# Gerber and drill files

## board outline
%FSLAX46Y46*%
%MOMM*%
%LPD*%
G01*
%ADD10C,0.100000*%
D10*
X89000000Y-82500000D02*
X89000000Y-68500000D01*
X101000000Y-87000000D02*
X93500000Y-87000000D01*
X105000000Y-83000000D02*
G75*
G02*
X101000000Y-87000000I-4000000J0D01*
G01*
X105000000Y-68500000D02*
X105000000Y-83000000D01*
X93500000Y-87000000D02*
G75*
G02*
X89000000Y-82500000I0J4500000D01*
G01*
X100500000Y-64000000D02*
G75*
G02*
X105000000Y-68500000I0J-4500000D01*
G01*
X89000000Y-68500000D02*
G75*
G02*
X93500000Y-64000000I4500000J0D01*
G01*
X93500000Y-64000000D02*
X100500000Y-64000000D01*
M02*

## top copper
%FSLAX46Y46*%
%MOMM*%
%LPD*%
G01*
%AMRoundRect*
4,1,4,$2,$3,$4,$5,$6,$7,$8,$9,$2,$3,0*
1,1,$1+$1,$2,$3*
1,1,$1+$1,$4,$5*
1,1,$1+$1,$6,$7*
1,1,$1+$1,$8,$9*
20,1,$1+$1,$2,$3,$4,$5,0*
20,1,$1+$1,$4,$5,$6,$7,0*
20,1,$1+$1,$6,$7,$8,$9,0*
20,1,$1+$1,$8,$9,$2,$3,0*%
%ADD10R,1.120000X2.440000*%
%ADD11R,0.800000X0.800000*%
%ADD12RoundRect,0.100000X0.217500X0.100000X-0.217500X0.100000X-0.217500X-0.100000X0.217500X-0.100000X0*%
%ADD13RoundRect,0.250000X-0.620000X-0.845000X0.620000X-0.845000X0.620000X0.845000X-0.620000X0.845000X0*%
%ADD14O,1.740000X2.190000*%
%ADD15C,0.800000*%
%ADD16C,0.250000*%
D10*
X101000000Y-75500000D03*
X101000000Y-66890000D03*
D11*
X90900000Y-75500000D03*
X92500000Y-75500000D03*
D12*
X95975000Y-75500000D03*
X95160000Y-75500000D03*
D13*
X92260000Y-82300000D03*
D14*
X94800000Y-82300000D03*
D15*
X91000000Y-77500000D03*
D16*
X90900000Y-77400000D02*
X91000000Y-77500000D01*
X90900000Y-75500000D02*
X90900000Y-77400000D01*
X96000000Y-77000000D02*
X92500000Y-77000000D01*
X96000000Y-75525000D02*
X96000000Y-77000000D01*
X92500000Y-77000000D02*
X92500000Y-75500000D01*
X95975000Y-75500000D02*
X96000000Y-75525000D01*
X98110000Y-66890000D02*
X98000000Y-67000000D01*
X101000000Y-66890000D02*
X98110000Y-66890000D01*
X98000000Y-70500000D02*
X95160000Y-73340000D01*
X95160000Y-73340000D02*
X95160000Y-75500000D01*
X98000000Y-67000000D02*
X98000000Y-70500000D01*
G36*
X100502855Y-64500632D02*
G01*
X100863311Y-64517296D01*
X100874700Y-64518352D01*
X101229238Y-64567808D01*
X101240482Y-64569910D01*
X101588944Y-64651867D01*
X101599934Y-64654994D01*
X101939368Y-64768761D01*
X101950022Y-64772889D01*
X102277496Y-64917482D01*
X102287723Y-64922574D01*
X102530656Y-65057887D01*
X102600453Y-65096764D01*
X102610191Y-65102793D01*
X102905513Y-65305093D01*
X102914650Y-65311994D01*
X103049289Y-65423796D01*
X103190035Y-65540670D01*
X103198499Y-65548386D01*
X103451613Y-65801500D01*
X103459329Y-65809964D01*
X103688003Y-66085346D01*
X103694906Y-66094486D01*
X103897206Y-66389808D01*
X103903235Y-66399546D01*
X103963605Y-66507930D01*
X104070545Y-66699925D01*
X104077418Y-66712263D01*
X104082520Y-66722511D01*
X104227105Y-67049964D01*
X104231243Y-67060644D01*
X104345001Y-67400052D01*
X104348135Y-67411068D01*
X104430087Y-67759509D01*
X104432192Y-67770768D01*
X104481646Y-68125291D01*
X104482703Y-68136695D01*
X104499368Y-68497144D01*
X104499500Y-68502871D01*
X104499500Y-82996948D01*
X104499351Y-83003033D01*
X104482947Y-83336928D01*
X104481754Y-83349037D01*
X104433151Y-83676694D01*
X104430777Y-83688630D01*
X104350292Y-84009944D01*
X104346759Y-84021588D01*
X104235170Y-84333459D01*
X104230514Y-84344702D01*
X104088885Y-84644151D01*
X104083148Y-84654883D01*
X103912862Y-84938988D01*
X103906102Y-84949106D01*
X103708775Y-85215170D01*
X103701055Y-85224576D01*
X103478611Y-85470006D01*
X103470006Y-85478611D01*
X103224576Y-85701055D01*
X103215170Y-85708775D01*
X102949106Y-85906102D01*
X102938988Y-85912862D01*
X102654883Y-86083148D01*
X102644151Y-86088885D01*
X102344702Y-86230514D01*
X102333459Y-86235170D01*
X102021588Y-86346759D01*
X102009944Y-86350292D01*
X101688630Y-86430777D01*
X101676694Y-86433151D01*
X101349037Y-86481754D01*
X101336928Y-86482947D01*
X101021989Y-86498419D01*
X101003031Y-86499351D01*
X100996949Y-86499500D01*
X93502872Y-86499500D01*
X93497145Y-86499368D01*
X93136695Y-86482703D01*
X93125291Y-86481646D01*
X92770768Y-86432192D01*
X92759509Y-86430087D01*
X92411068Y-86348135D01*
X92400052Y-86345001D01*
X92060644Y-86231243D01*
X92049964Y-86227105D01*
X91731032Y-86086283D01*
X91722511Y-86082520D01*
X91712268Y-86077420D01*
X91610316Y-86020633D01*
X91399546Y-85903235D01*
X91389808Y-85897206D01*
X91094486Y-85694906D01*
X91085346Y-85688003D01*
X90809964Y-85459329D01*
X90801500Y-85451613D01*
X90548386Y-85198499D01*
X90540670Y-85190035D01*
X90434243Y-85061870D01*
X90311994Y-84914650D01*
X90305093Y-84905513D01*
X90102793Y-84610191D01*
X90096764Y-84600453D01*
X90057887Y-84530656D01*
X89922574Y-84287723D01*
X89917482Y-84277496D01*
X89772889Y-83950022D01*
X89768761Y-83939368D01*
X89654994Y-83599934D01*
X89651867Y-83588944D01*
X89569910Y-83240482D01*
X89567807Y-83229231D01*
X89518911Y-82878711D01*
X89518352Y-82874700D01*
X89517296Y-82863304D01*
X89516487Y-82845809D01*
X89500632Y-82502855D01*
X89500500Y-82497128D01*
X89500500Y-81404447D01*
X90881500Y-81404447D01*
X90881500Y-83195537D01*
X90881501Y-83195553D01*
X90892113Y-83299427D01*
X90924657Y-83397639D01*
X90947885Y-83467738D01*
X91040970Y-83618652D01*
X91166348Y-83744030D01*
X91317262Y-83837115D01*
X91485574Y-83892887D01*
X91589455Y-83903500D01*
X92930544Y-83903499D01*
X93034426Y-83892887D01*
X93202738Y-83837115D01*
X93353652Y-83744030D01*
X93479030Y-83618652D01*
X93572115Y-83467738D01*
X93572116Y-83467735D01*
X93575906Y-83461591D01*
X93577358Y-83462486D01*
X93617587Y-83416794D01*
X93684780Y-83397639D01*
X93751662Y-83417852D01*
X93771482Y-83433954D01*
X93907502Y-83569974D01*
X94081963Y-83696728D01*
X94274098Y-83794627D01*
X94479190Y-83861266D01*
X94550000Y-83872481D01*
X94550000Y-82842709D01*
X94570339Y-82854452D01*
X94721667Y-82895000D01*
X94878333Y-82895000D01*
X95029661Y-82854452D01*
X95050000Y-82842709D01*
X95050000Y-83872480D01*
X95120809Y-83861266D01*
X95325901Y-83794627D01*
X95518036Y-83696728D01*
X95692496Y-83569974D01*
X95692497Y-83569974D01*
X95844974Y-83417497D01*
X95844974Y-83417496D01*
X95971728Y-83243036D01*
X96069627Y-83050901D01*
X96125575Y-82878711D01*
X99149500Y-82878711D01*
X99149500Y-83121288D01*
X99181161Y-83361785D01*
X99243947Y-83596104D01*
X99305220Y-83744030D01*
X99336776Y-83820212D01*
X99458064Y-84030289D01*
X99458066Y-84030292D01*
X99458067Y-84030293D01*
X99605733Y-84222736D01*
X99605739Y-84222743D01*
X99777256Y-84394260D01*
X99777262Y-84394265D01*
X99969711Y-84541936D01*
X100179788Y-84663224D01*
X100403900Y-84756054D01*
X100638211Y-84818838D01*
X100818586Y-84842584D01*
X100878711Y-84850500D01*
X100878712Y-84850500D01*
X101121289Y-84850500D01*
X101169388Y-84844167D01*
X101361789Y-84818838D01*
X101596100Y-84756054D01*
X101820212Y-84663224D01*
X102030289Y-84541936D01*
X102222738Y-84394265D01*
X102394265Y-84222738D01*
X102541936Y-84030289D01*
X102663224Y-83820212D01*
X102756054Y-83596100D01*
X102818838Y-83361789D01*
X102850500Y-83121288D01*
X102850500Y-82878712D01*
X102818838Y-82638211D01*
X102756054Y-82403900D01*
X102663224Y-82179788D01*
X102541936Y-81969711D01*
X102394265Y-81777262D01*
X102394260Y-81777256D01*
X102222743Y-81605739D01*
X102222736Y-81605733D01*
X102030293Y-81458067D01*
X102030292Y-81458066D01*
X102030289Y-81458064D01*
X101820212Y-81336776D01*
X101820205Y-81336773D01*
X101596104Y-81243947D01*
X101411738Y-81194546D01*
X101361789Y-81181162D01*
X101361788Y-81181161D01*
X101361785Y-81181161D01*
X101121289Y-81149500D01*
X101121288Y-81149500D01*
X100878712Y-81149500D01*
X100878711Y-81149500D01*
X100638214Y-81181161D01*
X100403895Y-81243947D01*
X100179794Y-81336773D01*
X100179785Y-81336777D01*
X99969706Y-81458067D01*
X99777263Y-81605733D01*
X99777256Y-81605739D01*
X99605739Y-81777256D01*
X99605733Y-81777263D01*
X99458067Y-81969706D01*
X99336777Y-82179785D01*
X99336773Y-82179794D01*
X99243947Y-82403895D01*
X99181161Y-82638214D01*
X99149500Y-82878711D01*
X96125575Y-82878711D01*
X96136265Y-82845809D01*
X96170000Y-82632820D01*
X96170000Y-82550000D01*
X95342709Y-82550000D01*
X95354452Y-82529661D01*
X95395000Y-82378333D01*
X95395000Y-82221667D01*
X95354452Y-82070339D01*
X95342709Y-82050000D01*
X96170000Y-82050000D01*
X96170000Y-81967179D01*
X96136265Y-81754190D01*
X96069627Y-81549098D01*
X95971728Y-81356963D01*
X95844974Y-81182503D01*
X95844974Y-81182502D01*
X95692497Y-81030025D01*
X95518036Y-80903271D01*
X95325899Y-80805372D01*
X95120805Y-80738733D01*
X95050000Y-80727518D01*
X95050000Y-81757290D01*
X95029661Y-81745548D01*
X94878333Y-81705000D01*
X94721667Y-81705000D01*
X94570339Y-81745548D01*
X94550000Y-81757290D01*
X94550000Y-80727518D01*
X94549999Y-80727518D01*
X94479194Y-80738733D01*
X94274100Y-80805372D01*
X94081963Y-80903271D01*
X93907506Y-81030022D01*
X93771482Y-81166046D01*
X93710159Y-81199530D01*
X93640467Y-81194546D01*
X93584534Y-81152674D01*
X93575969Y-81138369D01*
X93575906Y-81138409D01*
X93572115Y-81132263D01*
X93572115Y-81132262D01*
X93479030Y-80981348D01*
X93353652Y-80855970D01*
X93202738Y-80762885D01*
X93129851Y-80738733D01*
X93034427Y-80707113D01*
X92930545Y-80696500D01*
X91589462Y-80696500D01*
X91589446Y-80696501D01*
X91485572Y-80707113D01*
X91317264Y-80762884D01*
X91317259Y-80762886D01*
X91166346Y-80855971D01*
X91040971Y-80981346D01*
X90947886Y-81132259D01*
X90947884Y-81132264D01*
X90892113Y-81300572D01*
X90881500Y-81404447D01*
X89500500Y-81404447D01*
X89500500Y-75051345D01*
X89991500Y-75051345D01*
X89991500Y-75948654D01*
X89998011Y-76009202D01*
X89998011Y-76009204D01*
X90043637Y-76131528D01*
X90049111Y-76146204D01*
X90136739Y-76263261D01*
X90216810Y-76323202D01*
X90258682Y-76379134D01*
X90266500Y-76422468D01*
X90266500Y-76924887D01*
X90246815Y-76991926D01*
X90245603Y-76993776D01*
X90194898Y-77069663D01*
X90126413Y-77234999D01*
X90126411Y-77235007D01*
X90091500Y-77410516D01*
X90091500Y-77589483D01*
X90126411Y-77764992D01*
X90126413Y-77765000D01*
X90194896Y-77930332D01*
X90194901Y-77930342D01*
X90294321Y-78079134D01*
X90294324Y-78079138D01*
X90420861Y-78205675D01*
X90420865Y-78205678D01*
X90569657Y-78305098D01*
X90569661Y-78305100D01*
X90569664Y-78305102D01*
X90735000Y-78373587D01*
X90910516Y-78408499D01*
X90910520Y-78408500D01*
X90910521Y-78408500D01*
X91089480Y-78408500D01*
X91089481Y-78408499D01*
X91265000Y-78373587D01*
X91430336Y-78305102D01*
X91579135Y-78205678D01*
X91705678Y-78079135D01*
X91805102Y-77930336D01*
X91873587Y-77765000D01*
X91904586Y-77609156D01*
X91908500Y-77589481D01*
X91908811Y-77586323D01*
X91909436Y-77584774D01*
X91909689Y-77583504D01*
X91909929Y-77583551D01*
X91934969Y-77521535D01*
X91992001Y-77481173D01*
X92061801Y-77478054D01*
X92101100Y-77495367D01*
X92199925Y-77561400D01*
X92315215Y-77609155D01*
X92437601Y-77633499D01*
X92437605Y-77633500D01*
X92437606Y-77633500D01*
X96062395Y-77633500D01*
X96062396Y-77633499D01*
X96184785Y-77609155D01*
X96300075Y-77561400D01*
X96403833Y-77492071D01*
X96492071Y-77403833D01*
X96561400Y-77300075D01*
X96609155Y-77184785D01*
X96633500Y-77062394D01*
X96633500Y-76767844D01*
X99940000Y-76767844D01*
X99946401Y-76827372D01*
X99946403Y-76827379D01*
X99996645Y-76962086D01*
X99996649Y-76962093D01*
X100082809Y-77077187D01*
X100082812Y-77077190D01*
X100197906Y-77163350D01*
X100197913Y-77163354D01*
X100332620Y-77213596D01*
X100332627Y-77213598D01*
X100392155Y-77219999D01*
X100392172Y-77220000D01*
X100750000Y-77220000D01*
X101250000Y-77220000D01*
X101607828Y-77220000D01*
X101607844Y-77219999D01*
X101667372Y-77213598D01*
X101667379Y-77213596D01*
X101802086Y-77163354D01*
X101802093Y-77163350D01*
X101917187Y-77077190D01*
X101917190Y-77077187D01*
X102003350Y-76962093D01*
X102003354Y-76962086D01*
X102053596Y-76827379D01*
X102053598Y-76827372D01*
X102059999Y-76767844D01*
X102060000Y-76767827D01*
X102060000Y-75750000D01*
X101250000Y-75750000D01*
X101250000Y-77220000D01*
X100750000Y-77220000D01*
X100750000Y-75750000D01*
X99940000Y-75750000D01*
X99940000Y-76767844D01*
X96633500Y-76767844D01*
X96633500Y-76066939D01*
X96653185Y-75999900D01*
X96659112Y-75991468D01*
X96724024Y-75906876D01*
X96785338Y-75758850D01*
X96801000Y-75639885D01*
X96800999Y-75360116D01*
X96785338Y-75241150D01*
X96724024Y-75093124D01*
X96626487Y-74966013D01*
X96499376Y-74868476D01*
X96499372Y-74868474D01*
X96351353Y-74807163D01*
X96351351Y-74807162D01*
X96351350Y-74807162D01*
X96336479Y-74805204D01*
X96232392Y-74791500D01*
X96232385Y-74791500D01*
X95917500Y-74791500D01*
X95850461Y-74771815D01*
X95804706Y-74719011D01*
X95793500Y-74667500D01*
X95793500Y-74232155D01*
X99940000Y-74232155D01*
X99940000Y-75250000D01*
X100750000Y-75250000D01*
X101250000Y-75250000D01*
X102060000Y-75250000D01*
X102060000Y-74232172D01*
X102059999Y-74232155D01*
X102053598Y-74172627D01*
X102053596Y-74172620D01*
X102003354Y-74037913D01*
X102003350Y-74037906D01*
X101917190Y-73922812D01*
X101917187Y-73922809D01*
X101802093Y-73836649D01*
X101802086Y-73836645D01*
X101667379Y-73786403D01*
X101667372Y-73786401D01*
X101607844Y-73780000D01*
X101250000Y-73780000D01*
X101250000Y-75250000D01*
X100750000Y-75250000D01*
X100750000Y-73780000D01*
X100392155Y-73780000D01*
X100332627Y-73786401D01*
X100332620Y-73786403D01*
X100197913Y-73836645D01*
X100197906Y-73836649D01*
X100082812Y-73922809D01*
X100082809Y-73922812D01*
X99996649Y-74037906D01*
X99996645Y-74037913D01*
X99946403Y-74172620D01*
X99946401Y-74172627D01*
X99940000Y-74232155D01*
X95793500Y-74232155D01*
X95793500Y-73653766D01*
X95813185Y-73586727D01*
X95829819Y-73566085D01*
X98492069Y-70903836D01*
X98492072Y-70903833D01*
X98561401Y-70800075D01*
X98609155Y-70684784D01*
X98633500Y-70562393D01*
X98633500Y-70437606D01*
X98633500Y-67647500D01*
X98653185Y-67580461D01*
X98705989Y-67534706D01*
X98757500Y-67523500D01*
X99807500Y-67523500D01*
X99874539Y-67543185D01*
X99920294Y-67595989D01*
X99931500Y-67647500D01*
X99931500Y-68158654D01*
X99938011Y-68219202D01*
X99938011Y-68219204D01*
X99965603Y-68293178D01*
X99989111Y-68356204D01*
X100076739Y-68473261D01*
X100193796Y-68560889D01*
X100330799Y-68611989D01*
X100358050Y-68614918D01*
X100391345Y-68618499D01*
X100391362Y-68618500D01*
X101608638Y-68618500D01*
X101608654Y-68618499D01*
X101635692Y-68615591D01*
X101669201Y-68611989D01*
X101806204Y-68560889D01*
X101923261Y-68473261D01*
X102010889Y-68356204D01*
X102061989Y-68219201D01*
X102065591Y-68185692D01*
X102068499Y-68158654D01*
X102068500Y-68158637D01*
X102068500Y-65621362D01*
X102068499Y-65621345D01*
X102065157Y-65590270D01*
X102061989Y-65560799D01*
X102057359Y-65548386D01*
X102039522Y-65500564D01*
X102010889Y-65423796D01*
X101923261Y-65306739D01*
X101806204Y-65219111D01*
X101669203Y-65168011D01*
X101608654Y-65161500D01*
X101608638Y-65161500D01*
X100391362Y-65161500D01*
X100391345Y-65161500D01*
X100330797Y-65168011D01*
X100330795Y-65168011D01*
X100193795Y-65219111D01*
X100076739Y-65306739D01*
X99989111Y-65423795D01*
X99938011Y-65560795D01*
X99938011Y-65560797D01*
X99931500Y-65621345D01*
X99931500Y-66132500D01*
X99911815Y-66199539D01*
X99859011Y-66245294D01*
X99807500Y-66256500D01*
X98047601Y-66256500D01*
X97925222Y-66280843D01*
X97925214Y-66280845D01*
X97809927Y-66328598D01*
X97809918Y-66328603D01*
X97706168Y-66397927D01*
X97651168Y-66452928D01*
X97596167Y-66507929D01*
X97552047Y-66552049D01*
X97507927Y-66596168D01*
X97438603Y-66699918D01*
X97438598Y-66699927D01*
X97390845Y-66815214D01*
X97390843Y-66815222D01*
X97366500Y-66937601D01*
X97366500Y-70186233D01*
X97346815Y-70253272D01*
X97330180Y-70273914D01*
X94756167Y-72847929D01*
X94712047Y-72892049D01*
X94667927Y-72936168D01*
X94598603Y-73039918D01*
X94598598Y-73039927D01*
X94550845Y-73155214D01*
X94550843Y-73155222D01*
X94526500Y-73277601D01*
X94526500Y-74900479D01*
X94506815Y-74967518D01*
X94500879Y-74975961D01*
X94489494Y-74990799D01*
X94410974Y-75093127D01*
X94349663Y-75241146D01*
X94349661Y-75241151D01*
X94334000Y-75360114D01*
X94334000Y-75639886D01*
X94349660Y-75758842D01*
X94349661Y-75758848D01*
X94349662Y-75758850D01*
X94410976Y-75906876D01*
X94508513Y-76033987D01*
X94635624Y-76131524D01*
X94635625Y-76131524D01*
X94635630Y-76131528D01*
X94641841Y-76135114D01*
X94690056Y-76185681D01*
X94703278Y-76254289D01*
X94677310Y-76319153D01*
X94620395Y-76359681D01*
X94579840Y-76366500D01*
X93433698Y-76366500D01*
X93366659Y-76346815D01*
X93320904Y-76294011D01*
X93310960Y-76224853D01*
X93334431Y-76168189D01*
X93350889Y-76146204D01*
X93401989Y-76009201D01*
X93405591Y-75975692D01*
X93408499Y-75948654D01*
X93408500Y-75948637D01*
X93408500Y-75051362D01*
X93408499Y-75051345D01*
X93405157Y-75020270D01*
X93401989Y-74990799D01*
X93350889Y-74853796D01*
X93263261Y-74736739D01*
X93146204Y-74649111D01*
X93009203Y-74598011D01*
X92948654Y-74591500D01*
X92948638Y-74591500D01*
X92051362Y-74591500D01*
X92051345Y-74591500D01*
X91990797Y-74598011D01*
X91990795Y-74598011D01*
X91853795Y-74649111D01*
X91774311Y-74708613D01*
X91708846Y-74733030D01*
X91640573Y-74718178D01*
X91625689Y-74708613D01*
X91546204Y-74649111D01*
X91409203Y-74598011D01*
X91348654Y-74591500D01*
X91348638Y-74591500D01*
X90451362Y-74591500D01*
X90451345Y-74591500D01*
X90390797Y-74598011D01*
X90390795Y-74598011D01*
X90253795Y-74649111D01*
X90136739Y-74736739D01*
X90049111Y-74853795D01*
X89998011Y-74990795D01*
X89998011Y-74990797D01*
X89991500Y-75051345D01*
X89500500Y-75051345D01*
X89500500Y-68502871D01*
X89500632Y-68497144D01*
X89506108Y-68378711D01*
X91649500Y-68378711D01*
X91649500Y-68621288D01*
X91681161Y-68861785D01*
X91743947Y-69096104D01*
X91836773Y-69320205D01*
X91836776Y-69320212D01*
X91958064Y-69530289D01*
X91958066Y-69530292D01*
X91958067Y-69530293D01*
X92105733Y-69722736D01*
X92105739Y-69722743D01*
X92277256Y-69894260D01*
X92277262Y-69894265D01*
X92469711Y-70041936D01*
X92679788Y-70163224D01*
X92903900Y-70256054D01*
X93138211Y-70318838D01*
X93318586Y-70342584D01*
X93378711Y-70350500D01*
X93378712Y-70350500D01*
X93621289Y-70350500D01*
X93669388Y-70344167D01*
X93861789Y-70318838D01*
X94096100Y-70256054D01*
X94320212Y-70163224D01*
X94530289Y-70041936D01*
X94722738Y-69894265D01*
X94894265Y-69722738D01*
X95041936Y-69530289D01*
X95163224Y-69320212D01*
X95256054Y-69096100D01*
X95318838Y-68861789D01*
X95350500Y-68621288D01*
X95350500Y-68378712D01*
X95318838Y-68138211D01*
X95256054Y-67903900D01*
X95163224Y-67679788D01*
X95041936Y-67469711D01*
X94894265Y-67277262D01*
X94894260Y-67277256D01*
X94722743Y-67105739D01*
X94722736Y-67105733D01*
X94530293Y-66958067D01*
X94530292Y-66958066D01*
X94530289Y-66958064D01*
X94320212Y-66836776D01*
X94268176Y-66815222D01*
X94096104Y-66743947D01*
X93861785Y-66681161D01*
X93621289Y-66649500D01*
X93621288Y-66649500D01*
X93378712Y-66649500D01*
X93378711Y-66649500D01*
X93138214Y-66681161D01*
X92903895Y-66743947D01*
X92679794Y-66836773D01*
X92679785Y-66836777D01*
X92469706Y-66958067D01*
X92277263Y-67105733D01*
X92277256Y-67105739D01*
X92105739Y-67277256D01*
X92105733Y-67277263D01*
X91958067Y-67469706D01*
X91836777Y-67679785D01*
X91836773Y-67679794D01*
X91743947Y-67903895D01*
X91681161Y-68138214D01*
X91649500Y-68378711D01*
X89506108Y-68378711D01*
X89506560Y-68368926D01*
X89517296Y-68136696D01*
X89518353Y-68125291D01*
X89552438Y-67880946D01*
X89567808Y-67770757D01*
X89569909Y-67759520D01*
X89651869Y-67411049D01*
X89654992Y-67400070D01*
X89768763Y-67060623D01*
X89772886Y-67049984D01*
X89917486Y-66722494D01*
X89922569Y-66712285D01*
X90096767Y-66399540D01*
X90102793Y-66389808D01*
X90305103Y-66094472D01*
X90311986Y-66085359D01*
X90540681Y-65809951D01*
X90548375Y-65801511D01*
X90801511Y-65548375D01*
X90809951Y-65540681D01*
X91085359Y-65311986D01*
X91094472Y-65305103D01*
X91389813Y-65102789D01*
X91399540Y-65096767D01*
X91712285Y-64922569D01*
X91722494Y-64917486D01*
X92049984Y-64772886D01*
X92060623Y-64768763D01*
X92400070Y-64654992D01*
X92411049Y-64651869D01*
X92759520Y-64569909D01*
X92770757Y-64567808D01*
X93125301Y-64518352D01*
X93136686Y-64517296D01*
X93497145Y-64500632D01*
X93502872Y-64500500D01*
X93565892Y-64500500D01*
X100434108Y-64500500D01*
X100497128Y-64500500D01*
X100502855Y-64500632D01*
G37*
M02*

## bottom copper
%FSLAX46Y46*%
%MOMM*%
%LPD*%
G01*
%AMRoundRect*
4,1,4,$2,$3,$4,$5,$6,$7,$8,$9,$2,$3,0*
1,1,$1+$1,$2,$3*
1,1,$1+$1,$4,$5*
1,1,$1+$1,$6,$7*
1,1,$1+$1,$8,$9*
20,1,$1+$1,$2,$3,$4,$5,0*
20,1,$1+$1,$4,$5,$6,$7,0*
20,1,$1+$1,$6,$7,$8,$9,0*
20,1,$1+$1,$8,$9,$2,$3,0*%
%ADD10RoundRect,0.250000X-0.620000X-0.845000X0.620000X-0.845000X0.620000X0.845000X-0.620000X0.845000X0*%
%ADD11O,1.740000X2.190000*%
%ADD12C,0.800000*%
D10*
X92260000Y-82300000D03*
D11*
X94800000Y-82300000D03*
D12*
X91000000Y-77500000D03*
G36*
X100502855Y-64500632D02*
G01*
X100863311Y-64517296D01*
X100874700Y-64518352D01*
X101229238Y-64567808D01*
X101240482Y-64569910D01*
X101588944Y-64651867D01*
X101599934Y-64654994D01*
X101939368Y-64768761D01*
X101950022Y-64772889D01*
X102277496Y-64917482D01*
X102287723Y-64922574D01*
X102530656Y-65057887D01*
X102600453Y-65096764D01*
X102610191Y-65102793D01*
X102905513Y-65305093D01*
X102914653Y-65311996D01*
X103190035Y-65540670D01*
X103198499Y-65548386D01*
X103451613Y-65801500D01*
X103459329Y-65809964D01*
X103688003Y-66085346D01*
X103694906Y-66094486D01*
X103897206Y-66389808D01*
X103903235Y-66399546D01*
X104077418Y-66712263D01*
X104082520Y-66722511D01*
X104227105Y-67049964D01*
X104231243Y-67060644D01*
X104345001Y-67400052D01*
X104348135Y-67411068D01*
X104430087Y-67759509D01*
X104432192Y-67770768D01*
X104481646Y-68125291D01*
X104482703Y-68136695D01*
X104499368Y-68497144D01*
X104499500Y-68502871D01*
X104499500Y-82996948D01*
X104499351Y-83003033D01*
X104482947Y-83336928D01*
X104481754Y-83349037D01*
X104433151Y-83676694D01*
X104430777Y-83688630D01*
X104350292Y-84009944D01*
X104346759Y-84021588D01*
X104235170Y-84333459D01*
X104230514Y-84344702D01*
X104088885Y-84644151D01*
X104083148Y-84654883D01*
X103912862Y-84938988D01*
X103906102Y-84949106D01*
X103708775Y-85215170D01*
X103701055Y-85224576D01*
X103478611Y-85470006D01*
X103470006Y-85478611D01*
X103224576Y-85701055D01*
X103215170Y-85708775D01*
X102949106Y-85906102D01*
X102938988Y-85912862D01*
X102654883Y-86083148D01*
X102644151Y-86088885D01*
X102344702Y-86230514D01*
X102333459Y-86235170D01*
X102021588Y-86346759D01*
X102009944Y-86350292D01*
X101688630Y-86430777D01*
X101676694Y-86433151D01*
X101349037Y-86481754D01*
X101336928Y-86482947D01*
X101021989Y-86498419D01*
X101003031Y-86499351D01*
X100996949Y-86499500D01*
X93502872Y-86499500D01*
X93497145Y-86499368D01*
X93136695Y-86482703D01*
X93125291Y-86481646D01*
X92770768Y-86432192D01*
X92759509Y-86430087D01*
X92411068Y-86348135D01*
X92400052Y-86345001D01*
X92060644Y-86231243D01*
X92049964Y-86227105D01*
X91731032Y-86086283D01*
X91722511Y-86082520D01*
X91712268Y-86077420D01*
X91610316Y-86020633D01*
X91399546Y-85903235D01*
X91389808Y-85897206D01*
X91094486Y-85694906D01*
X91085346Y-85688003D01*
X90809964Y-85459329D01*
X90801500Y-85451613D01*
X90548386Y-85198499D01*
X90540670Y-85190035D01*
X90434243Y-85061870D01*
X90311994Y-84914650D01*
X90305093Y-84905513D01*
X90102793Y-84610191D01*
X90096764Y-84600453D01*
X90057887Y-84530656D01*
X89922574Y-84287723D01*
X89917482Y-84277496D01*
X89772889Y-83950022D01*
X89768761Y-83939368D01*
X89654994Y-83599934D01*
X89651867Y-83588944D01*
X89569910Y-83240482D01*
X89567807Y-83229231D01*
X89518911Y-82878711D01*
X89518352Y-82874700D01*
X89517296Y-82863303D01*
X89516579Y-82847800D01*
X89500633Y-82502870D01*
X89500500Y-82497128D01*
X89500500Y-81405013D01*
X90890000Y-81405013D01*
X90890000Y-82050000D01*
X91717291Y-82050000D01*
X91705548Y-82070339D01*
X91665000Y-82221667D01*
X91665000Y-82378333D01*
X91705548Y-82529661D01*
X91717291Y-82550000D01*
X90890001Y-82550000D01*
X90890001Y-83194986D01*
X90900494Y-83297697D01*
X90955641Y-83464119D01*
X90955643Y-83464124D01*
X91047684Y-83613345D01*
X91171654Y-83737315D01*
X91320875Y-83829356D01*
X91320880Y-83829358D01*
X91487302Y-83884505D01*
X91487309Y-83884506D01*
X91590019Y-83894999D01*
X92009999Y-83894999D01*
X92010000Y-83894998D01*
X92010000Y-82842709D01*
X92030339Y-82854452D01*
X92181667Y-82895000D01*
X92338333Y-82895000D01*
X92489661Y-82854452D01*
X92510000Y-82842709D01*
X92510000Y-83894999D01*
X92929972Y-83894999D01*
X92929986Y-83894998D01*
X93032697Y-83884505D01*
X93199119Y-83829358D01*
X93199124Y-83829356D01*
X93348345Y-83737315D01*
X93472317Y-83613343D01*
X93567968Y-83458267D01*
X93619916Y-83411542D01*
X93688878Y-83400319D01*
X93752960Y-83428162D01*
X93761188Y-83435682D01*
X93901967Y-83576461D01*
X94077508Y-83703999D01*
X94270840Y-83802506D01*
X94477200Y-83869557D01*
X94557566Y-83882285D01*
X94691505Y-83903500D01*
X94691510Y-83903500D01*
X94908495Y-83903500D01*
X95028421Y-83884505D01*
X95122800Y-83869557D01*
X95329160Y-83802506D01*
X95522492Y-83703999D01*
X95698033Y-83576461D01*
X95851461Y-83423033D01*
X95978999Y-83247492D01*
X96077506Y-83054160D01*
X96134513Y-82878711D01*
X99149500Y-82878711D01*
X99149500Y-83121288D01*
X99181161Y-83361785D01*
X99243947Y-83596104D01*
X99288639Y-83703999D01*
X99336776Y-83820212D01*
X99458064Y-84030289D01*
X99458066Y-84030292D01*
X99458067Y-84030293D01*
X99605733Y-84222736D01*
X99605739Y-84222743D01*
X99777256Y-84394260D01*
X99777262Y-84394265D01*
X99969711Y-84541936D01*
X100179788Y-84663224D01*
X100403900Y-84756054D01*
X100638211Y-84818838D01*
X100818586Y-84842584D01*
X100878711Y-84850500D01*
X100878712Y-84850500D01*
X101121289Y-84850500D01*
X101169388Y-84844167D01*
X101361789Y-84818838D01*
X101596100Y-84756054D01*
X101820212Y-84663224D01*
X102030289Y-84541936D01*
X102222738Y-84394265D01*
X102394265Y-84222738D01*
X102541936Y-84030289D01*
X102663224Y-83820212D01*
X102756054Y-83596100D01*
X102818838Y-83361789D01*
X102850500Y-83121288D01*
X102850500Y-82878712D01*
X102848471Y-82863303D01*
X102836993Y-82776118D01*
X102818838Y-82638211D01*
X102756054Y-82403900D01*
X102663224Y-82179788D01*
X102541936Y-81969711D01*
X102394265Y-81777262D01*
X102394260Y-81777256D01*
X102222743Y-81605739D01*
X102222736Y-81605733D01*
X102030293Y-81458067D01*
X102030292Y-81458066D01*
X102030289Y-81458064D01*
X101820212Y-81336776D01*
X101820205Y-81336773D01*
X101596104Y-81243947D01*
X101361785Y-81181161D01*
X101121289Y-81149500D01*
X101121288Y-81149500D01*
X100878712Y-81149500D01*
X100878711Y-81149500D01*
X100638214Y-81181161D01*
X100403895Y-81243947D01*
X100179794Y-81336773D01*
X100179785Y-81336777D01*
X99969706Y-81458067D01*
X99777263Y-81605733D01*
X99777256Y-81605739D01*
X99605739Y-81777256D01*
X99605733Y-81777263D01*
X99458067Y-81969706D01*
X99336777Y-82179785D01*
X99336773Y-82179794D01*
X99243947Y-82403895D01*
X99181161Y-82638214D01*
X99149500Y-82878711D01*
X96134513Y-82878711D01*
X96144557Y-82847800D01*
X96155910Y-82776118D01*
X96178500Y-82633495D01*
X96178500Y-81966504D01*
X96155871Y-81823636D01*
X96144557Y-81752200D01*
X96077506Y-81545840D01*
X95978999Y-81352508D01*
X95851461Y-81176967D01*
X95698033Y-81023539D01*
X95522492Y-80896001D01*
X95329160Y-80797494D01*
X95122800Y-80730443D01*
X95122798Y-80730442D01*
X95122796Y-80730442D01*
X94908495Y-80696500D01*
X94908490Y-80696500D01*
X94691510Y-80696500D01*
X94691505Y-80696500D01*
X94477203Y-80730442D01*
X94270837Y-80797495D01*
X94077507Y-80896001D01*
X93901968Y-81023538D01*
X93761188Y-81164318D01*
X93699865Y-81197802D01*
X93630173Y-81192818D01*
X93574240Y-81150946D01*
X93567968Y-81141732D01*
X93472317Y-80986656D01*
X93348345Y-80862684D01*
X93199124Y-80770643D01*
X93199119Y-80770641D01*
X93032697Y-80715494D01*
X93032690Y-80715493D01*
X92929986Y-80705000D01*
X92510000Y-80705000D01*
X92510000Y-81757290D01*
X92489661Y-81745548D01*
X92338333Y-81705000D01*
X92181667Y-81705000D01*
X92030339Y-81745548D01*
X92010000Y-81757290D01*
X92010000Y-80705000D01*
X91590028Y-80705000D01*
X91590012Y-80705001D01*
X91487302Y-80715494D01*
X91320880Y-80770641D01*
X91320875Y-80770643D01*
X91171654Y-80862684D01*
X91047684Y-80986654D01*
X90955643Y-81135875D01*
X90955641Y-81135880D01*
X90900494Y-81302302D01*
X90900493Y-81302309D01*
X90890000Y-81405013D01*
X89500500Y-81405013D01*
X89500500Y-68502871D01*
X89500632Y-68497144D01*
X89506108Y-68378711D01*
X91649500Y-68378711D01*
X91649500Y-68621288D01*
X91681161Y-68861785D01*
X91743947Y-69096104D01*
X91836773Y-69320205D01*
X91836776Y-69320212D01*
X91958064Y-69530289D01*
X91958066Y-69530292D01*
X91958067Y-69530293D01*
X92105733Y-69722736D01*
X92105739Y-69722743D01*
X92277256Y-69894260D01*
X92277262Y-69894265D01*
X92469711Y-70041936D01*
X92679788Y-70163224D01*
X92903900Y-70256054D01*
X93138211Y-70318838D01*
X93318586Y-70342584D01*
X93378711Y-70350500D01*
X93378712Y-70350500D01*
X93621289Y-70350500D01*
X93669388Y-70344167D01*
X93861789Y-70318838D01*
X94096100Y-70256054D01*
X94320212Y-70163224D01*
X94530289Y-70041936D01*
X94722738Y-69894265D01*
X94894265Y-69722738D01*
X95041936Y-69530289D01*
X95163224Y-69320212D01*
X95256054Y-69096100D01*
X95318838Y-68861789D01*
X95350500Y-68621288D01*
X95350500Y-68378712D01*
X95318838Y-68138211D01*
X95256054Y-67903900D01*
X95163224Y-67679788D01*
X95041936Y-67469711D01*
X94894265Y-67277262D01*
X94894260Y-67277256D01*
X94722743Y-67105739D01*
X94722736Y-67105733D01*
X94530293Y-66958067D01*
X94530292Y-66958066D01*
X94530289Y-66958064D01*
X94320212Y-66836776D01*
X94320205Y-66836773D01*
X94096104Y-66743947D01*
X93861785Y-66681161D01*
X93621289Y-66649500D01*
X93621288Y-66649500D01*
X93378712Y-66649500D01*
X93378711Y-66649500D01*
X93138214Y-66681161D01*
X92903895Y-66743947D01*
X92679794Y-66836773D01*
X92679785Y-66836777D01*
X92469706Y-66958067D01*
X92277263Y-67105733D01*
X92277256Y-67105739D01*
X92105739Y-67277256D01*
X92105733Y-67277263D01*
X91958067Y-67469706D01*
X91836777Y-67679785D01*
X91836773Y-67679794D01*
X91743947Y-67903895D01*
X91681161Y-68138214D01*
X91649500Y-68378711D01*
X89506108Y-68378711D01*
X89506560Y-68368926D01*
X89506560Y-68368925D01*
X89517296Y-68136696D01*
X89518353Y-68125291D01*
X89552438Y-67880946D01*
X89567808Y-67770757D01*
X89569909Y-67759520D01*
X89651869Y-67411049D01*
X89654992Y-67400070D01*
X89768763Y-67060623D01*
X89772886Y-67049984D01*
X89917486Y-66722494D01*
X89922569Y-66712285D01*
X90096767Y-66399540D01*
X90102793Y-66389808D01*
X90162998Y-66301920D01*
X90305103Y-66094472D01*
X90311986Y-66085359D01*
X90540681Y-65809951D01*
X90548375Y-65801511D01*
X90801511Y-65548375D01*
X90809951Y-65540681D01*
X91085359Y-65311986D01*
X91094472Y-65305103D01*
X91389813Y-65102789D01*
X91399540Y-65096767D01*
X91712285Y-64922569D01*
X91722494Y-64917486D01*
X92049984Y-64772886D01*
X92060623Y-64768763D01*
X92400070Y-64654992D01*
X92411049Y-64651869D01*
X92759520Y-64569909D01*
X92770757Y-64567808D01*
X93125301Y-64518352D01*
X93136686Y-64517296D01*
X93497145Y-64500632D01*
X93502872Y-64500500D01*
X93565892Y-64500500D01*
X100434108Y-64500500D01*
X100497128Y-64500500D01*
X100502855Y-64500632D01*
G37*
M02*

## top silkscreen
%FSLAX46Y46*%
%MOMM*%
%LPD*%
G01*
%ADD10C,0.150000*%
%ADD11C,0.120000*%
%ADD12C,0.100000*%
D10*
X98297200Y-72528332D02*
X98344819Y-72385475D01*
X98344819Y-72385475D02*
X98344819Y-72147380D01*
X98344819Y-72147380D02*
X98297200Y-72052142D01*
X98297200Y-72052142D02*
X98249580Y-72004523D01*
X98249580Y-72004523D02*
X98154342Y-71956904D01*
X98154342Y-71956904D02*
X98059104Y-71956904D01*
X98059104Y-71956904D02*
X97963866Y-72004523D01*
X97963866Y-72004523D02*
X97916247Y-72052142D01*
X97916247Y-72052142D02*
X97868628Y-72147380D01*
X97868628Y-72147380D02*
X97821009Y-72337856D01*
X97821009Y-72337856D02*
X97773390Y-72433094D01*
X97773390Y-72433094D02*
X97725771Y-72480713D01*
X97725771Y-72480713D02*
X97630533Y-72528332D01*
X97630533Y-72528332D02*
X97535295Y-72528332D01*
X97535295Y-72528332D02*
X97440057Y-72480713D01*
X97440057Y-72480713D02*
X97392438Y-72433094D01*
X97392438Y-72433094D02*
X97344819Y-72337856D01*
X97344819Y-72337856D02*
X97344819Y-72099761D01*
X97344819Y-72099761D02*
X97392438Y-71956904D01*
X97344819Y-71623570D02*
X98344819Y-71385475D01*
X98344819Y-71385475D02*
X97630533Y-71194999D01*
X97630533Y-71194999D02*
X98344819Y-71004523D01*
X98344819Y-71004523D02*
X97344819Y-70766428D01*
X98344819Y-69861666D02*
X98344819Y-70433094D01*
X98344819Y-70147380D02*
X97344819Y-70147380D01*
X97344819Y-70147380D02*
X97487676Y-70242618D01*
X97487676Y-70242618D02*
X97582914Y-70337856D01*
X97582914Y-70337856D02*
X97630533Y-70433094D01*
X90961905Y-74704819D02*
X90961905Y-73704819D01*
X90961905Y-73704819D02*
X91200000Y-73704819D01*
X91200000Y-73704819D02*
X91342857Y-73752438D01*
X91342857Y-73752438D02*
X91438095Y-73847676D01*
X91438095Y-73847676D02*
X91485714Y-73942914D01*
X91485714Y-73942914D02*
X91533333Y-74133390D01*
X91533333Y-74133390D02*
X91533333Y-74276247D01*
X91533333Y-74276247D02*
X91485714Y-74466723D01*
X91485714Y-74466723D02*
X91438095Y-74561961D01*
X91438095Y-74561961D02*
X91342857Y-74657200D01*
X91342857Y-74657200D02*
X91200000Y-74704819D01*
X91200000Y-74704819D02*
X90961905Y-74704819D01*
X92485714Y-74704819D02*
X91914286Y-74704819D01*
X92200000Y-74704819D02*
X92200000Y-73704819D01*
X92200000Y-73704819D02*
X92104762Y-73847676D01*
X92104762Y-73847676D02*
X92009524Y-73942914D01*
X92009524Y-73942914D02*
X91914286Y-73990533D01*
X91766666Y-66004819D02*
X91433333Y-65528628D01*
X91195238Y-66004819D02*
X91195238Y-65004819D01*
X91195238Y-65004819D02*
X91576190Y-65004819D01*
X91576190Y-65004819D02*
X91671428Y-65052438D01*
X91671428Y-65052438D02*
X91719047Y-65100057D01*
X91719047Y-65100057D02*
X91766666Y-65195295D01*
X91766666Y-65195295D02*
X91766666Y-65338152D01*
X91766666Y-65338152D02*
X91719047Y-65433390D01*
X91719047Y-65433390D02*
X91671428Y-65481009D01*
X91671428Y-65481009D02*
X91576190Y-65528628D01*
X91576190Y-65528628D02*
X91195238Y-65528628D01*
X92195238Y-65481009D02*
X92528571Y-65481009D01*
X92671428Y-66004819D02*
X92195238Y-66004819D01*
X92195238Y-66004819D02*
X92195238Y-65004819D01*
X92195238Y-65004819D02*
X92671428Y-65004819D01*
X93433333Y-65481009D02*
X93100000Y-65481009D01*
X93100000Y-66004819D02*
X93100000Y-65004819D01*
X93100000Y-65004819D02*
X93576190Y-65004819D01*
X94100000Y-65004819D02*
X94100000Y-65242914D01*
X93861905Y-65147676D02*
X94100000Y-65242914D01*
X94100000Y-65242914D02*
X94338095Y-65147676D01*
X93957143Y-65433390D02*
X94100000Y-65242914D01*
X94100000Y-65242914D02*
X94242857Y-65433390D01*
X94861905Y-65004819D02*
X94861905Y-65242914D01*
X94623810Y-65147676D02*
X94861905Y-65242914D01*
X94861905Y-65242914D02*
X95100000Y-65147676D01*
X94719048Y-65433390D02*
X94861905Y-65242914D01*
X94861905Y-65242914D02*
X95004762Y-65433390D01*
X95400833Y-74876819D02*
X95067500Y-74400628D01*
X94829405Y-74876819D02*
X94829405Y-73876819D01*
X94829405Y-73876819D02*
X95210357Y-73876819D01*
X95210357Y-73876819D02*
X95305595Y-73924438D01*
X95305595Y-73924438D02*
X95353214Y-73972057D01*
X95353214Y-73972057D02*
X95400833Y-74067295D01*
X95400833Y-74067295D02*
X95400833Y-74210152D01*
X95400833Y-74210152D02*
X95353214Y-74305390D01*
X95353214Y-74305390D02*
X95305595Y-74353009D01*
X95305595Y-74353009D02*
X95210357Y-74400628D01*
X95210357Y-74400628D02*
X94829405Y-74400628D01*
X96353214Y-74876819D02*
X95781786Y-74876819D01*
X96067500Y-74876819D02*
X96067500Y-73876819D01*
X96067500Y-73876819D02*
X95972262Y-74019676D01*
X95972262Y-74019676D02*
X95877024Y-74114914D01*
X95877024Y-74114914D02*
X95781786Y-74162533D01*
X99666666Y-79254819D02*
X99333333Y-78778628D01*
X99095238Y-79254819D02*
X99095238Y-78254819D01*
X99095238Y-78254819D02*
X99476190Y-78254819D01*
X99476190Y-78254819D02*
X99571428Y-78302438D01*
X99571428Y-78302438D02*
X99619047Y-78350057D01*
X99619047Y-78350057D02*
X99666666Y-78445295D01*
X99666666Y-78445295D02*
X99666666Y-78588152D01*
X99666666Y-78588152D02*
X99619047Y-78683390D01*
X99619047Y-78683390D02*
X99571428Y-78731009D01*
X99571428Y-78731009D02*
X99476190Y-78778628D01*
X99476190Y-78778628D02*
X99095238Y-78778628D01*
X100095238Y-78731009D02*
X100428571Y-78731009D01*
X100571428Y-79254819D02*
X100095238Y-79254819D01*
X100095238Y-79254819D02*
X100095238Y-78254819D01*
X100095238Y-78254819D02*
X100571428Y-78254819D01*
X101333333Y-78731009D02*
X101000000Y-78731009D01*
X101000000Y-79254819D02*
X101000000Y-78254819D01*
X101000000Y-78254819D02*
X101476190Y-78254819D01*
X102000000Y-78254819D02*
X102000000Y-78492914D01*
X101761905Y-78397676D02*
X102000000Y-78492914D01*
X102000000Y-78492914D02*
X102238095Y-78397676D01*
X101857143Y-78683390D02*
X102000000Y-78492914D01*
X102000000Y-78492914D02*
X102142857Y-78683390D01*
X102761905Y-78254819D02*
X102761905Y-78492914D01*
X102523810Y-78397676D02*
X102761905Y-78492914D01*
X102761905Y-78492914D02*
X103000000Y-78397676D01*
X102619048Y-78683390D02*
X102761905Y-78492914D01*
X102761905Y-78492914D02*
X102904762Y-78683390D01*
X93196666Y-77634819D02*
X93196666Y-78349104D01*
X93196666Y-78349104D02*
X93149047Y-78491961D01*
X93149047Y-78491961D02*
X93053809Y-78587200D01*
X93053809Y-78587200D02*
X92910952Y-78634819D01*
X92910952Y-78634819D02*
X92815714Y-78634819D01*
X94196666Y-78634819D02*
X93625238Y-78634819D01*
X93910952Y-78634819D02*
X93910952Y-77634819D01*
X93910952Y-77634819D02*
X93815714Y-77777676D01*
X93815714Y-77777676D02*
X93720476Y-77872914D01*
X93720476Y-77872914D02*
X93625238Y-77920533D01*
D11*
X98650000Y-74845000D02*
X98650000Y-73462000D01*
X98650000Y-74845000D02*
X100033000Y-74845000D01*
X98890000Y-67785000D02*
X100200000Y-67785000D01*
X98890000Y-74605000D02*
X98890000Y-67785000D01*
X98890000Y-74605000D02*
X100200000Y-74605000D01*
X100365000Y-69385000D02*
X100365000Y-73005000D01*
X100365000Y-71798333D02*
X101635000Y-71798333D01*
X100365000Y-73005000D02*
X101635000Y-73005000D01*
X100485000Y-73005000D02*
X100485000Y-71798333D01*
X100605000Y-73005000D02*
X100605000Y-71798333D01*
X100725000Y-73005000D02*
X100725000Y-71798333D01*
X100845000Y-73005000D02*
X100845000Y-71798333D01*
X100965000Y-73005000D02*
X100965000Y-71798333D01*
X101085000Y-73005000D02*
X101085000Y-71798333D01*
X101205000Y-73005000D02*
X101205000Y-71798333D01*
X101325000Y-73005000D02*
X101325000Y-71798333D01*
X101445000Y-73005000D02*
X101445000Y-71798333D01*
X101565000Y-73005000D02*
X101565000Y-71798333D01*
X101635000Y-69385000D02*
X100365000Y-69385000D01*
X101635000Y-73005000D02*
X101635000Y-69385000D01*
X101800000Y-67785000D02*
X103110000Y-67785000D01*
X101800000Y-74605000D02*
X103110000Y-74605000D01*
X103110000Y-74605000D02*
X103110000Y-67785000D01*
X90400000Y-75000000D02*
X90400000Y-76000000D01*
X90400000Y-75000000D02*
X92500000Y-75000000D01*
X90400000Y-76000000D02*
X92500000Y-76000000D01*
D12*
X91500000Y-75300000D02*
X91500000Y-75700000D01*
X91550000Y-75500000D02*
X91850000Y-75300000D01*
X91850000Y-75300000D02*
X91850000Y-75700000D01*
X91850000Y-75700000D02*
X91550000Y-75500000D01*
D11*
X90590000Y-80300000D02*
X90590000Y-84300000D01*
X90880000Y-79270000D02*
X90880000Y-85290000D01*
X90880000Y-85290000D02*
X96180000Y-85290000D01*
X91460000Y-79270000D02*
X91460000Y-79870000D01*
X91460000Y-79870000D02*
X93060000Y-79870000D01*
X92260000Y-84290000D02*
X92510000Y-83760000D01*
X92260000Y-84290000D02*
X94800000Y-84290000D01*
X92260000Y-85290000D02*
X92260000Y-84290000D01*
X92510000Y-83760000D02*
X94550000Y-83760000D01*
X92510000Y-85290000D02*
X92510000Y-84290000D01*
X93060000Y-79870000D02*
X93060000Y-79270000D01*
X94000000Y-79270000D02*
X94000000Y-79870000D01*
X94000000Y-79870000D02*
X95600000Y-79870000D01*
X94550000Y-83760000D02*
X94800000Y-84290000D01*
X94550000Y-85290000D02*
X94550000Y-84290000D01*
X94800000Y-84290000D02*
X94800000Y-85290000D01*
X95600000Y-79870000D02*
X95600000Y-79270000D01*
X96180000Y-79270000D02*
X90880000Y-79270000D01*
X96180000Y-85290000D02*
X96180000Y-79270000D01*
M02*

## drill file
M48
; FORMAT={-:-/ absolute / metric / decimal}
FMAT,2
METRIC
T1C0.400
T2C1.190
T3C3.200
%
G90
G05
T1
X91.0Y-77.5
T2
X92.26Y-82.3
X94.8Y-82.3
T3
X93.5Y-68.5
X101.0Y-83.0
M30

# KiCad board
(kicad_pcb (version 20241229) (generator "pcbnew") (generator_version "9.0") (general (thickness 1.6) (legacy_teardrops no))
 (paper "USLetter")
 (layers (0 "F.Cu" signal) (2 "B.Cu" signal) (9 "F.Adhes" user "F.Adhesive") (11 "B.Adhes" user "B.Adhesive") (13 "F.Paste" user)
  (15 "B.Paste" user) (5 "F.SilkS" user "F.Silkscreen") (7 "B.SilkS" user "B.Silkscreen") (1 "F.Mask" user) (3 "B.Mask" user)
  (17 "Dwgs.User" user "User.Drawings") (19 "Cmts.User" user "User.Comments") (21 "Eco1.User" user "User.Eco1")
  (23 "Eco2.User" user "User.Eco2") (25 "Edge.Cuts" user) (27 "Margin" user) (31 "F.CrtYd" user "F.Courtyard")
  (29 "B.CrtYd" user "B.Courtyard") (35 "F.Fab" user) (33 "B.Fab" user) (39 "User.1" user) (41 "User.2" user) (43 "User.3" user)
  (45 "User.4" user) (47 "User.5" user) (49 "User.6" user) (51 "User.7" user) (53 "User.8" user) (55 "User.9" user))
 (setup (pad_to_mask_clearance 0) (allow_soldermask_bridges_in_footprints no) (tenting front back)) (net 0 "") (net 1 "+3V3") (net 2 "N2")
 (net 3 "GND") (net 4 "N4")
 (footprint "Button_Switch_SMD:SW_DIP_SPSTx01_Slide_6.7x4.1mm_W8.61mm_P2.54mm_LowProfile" (layer "F.Cu") (at 101 71.195 90)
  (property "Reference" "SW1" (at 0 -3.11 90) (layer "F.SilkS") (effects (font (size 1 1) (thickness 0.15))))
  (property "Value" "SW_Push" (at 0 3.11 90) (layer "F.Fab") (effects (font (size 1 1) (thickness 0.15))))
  (fp_line (start -3.65 -2.35) (end -2.267 -2.35) (stroke (width 0.12) (type solid)) (layer "F.SilkS"))
  (fp_line (start -3.65 -2.35) (end -3.65 -0.967) (stroke (width 0.12) (type solid)) (layer "F.SilkS"))
  (fp_line (start 3.41 -2.11) (end 3.41 -0.8) (stroke (width 0.12) (type solid)) (layer "F.SilkS"))
  (fp_line (start -3.41 -2.11) (end 3.41 -2.11) (stroke (width 0.12) (type solid)) (layer "F.SilkS"))
  (fp_line (start -3.41 -2.11) (end -3.41 -0.8) (stroke (width 0.12) (type solid)) (layer "F.SilkS"))
  (fp_line (start 1.81 -0.635) (end -1.81 -0.635) (stroke (width 0.12) (type solid)) (layer "F.SilkS"))
  (fp_line (start -0.603333 -0.635) (end -0.603333 0.635) (stroke (width 0.12) (type solid)) (layer "F.SilkS"))
  (fp_line (start -1.81 -0.635) (end -1.81 0.635) (stroke (width 0.12) (type solid)) (layer "F.SilkS"))
  (fp_line (start -1.81 -0.515) (end -0.603333 -0.515) (stroke (width 0.12) (type solid)) (layer "F.SilkS"))
  (fp_line (start -1.81 -0.395) (end -0.603333 -0.395) (stroke (width 0.12) (type solid)) (layer "F.SilkS"))
  (fp_line (start -1.81 -0.275) (end -0.603333 -0.275) (stroke (width 0.12) (type solid)) (layer "F.SilkS"))
  (fp_line (start -1.81 -0.155) (end -0.603333 -0.155) (stroke (width 0.12) (type solid)) (layer "F.SilkS"))
  (fp_line (start -1.81 -0.035) (end -0.603333 -0.035) (stroke (width 0.12) (type solid)) (layer "F.SilkS"))
  (fp_line (start -1.81 0.085) (end -0.603333 0.085) (stroke (width 0.12) (type solid)) (layer "F.SilkS"))
  (fp_line (start -1.81 0.205) (end -0.603333 0.205) (stroke (width 0.12) (type solid)) (layer "F.SilkS"))
  (fp_line (start -1.81 0.325) (end -0.603333 0.325) (stroke (width 0.12) (type solid)) (layer "F.SilkS"))
  (fp_line (start -1.81 0.445) (end -0.603333 0.445) (stroke (width 0.12) (type solid)) (layer "F.SilkS"))
  (fp_line (start -1.81 0.565) (end -0.603333 0.565) (stroke (width 0.12) (type solid)) (layer "F.SilkS"))
  (fp_line (start 1.81 0.635) (end 1.81 -0.635) (stroke (width 0.12) (type solid)) (layer "F.SilkS"))
  (fp_line (start -1.81 0.635) (end 1.81 0.635) (stroke (width 0.12) (type solid)) (layer "F.SilkS"))
  (fp_line (start 3.41 0.8) (end 3.41 2.11) (stroke (width 0.12) (type solid)) (layer "F.SilkS"))
  (fp_line (start -3.41 0.8) (end -3.41 2.11) (stroke (width 0.12) (type solid)) (layer "F.SilkS"))
  (fp_line (start -3.41 2.11) (end 3.41 2.11) (stroke (width 0.12) (type solid)) (layer "F.SilkS"))
  (pad "1" smd rect (at -4.305 0 90) (size 2.44 1.12) (layers "F.Cu" "F.Mask" "F.Paste") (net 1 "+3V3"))
  (pad "2" smd rect (at 4.305 0 90) (size 2.44 1.12) (layers "F.Cu" "F.Mask" "F.Paste") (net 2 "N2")))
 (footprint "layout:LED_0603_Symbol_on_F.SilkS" (layer "F.Cu") (at 91.7 75.5)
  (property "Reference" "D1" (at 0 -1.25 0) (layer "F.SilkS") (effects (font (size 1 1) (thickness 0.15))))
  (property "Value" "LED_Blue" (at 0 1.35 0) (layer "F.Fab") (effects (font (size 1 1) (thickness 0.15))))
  (fp_line (start -1.3 -0.5) (end -1.3 0.5) (stroke (width 0.12) (type solid)) (layer "F.SilkS"))
  (fp_line (start -1.3 -0.5) (end 0.8 -0.5) (stroke (width 0.12) (type solid)) (layer "F.SilkS"))
  (fp_line (start -1.3 0.5) (end 0.8 0.5) (stroke (width 0.12) (type solid)) (layer "F.SilkS"))
  (fp_line (start -0.2 -0.2) (end -0.2 0.2) (stroke (width 0.1) (type solid)) (layer "F.SilkS"))
  (fp_line (start -0.15 0) (end 0.15 -0.2) (stroke (width 0.1) (type solid)) (layer "F.SilkS"))
  (fp_line (start 0.15 -0.2) (end 0.15 0.2) (stroke (width 0.1) (type solid)) (layer "F.SilkS"))
  (fp_line (start 0.15 0.2) (end -0.15 0) (stroke (width 0.1) (type solid)) (layer "F.SilkS"))
  (pad "1" smd rect (at -0.8 0 180) (size 0.8 0.8) (layers "F.Cu" "F.Mask" "F.Paste") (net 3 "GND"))
  (pad "2" smd rect (at 0.8 0 180) (size 0.8 0.8) (layers "F.Cu" "F.Mask" "F.Paste") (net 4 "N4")))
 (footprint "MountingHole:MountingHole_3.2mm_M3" (layer "F.Cu") (at 93.5 68.5)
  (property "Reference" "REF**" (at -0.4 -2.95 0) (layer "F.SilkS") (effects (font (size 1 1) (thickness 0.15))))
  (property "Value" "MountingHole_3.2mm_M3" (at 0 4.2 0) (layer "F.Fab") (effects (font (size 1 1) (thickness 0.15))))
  (pad "" np_thru_hole circle (at 0 0) (size 3.2 3.2) (drill 3.2) (layers "*.Cu" "*.Mask")))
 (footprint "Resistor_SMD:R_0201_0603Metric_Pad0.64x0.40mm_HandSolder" (layer "F.Cu") (at 95.5675 75.5 180)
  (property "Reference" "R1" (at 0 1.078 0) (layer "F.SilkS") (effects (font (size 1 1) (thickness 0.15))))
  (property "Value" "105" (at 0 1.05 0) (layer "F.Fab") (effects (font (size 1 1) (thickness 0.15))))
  (pad "" smd roundrect (at -0.4325 0 180) (size 0.458 0.36) (layers "F.Paste") (roundrect_rratio 0.25))
  (pad "" smd roundrect (at 0.4325 0 180) (size 0.458 0.36) (layers "F.Paste") (roundrect_rratio 0.25))
  (pad "1" smd roundrect (at -0.4075 0 180) (size 0.635 0.4) (layers "F.Cu" "F.Mask") (roundrect_rratio 0.25) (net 4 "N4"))
  (pad "2" smd roundrect (at 0.4075 0 180) (size 0.635 0.4) (layers "F.Cu" "F.Mask") (roundrect_rratio 0.25) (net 2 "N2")))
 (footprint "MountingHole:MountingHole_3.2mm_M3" (layer "F.Cu") (at 101 83)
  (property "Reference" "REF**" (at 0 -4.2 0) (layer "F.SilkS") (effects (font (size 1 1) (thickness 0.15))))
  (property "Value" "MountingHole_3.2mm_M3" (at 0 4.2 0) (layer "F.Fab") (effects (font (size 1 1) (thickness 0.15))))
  (pad "" np_thru_hole circle (at 0 0) (size 3.2 3.2) (drill 3.2) (layers "*.Cu" "*.Mask")))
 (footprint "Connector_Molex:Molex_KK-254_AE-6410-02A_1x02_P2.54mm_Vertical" (layer "F.Cu") (at 92.26 82.3)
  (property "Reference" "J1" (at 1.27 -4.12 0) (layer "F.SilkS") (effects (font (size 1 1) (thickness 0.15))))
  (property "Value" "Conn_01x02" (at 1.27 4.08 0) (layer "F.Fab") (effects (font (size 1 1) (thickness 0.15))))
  (fp_line (start -1.67 -2) (end -1.67 2) (stroke (width 0.12) (type solid)) (layer "F.SilkS"))
  (fp_line (start -1.38 -3.03) (end -1.38 2.99) (stroke (width 0.12) (type solid)) (layer "F.SilkS"))
  (fp_line (start -1.38 2.99) (end 3.92 2.99) (stroke (width 0.12) (type solid)) (layer "F.SilkS"))
  (fp_line (start -0.8 -3.03) (end -0.8 -2.43) (stroke (width 0.12) (type solid)) (layer "F.SilkS"))
  (fp_line (start -0.8 -2.43) (end 0.8 -2.43) (stroke (width 0.12) (type solid)) (layer "F.SilkS"))
  (fp_line (start 0 1.99) (end 0.25 1.46) (stroke (width 0.12) (type solid)) (layer "F.SilkS"))
  (fp_line (start 0 1.99) (end 2.54 1.99) (stroke (width 0.12) (type solid)) (layer "F.SilkS"))
  (fp_line (start 0 2.99) (end 0 1.99) (stroke (width 0.12) (type solid)) (layer "F.SilkS"))
  (fp_line (start 0.25 1.46) (end 2.29 1.46) (stroke (width 0.12) (type solid)) (layer "F.SilkS"))
  (fp_line (start 0.25 2.99) (end 0.25 1.99) (stroke (width 0.12) (type solid)) (layer "F.SilkS"))
  (fp_line (start 0.8 -2.43) (end 0.8 -3.03) (stroke (width 0.12) (type solid)) (layer "F.SilkS"))
  (fp_line (start 1.74 -3.03) (end 1.74 -2.43) (stroke (width 0.12) (type solid)) (layer "F.SilkS"))
  (fp_line (start 1.74 -2.43) (end 3.34 -2.43) (stroke (width 0.12) (type solid)) (layer "F.SilkS"))
  (fp_line (start 2.29 1.46) (end 2.54 1.99) (stroke (width 0.12) (type solid)) (layer "F.SilkS"))
  (fp_line (start 2.29 2.99) (end 2.29 1.99) (stroke (width 0.12) (type solid)) (layer "F.SilkS"))
  (fp_line (start 2.54 1.99) (end 2.54 2.99) (stroke (width 0.12) (type solid)) (layer "F.SilkS"))
  (fp_line (start 3.34 -2.43) (end 3.34 -3.03) (stroke (width 0.12) (type solid)) (layer "F.SilkS"))
  (fp_line (start 3.92 -3.03) (end -1.38 -3.03) (stroke (width 0.12) (type solid)) (layer "F.SilkS"))
  (fp_line (start 3.92 2.99) (end 3.92 -3.03) (stroke (width 0.12) (type solid)) (layer "F.SilkS"))
  (pad "1" thru_hole roundrect (at 0 0) (size 1.74 2.19) (drill 1.19) (layers "*.Cu" "*.Mask") (remove_unused_layers no)
   (roundrect_rratio 0.143678) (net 3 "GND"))
  (pad "2" thru_hole oval (at 2.54 0) (size 1.74 2.19) (drill 1.19) (layers "*.Cu" "*.Mask") (remove_unused_layers no) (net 1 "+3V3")))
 (gr_line (start 89 82.5) (end 89 68.5) (stroke (width 0.1) (type default)) (layer "Edge.Cuts"))
 (gr_line (start 101 87) (end 93.5 87) (stroke (width 0.1) (type default)) (layer "Edge.Cuts"))
 (gr_arc (start 105 83) (mid 103.828427 85.828427) (end 101 87) (stroke (width 0.1) (type default)) (layer "Edge.Cuts"))
 (gr_line (start 105 68.5) (end 105 83) (stroke (width 0.1) (type default)) (layer "Edge.Cuts"))
 (gr_arc (start 93.5 87) (mid 90.318019 85.681981) (end 89 82.5) (stroke (width 0.1) (type default)) (layer "Edge.Cuts"))
 (gr_arc (start 100.5 64) (mid 103.681981 65.318019) (end 105 68.5) (stroke (width 0.1) (type default)) (layer "Edge.Cuts"))
 (gr_arc (start 89 68.5) (mid 90.318019 65.318019) (end 93.5 64) (stroke (width 0.1) (type default)) (layer "Edge.Cuts"))
 (gr_line (start 93.5 64) (end 100.5 64) (stroke (width 0.1) (type default)) (layer "Edge.Cuts"))
 (segment (start 90.9 77.4) (end 91 77.5) (width 0.25) (layer "F.Cu") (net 3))
 (segment (start 90.9 75.5) (end 90.9 77.4) (width 0.25) (layer "F.Cu") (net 3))
 (via (at 91 77.5) (size 0.8) (drill 0.4) (layers "F.Cu" "B.Cu") (free yes) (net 3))
 (segment (start 96 77) (end 92.5 77) (width 0.25) (layer "F.Cu") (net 4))
 (segment (start 96 75.525) (end 96 77) (width 0.25) (layer "F.Cu") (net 4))
 (segment (start 92.5 77) (end 92.5 75.5) (width 0.25) (layer "F.Cu") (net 4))
 (segment (start 95.975 75.5) (end 96 75.525) (width 0.25) (layer "F.Cu") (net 4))
 (segment (start 98.11 66.89) (end 98 67) (width 0.25) (layer "F.Cu") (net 2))
 (segment (start 101 66.89) (end 98.11 66.89) (width 0.25) (layer "F.Cu") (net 2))
 (segment (start 98 70.5) (end 95.16 73.34) (width 0.25) (layer "F.Cu") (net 2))
 (segment (start 95.16 73.34) (end 95.16 75.5) (width 0.25) (layer "F.Cu") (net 2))
 (segment (start 98 67) (end 98 70.5) (width 0.25) (layer "F.Cu") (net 2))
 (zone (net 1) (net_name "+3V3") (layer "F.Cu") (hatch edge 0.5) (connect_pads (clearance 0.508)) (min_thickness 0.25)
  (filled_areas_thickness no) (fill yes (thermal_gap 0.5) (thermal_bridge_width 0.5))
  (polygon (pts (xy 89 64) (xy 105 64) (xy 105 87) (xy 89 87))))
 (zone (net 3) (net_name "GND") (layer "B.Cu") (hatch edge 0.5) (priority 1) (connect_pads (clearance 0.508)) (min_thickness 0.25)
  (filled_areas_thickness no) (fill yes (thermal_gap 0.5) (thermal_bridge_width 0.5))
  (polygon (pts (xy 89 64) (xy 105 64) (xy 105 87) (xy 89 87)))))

